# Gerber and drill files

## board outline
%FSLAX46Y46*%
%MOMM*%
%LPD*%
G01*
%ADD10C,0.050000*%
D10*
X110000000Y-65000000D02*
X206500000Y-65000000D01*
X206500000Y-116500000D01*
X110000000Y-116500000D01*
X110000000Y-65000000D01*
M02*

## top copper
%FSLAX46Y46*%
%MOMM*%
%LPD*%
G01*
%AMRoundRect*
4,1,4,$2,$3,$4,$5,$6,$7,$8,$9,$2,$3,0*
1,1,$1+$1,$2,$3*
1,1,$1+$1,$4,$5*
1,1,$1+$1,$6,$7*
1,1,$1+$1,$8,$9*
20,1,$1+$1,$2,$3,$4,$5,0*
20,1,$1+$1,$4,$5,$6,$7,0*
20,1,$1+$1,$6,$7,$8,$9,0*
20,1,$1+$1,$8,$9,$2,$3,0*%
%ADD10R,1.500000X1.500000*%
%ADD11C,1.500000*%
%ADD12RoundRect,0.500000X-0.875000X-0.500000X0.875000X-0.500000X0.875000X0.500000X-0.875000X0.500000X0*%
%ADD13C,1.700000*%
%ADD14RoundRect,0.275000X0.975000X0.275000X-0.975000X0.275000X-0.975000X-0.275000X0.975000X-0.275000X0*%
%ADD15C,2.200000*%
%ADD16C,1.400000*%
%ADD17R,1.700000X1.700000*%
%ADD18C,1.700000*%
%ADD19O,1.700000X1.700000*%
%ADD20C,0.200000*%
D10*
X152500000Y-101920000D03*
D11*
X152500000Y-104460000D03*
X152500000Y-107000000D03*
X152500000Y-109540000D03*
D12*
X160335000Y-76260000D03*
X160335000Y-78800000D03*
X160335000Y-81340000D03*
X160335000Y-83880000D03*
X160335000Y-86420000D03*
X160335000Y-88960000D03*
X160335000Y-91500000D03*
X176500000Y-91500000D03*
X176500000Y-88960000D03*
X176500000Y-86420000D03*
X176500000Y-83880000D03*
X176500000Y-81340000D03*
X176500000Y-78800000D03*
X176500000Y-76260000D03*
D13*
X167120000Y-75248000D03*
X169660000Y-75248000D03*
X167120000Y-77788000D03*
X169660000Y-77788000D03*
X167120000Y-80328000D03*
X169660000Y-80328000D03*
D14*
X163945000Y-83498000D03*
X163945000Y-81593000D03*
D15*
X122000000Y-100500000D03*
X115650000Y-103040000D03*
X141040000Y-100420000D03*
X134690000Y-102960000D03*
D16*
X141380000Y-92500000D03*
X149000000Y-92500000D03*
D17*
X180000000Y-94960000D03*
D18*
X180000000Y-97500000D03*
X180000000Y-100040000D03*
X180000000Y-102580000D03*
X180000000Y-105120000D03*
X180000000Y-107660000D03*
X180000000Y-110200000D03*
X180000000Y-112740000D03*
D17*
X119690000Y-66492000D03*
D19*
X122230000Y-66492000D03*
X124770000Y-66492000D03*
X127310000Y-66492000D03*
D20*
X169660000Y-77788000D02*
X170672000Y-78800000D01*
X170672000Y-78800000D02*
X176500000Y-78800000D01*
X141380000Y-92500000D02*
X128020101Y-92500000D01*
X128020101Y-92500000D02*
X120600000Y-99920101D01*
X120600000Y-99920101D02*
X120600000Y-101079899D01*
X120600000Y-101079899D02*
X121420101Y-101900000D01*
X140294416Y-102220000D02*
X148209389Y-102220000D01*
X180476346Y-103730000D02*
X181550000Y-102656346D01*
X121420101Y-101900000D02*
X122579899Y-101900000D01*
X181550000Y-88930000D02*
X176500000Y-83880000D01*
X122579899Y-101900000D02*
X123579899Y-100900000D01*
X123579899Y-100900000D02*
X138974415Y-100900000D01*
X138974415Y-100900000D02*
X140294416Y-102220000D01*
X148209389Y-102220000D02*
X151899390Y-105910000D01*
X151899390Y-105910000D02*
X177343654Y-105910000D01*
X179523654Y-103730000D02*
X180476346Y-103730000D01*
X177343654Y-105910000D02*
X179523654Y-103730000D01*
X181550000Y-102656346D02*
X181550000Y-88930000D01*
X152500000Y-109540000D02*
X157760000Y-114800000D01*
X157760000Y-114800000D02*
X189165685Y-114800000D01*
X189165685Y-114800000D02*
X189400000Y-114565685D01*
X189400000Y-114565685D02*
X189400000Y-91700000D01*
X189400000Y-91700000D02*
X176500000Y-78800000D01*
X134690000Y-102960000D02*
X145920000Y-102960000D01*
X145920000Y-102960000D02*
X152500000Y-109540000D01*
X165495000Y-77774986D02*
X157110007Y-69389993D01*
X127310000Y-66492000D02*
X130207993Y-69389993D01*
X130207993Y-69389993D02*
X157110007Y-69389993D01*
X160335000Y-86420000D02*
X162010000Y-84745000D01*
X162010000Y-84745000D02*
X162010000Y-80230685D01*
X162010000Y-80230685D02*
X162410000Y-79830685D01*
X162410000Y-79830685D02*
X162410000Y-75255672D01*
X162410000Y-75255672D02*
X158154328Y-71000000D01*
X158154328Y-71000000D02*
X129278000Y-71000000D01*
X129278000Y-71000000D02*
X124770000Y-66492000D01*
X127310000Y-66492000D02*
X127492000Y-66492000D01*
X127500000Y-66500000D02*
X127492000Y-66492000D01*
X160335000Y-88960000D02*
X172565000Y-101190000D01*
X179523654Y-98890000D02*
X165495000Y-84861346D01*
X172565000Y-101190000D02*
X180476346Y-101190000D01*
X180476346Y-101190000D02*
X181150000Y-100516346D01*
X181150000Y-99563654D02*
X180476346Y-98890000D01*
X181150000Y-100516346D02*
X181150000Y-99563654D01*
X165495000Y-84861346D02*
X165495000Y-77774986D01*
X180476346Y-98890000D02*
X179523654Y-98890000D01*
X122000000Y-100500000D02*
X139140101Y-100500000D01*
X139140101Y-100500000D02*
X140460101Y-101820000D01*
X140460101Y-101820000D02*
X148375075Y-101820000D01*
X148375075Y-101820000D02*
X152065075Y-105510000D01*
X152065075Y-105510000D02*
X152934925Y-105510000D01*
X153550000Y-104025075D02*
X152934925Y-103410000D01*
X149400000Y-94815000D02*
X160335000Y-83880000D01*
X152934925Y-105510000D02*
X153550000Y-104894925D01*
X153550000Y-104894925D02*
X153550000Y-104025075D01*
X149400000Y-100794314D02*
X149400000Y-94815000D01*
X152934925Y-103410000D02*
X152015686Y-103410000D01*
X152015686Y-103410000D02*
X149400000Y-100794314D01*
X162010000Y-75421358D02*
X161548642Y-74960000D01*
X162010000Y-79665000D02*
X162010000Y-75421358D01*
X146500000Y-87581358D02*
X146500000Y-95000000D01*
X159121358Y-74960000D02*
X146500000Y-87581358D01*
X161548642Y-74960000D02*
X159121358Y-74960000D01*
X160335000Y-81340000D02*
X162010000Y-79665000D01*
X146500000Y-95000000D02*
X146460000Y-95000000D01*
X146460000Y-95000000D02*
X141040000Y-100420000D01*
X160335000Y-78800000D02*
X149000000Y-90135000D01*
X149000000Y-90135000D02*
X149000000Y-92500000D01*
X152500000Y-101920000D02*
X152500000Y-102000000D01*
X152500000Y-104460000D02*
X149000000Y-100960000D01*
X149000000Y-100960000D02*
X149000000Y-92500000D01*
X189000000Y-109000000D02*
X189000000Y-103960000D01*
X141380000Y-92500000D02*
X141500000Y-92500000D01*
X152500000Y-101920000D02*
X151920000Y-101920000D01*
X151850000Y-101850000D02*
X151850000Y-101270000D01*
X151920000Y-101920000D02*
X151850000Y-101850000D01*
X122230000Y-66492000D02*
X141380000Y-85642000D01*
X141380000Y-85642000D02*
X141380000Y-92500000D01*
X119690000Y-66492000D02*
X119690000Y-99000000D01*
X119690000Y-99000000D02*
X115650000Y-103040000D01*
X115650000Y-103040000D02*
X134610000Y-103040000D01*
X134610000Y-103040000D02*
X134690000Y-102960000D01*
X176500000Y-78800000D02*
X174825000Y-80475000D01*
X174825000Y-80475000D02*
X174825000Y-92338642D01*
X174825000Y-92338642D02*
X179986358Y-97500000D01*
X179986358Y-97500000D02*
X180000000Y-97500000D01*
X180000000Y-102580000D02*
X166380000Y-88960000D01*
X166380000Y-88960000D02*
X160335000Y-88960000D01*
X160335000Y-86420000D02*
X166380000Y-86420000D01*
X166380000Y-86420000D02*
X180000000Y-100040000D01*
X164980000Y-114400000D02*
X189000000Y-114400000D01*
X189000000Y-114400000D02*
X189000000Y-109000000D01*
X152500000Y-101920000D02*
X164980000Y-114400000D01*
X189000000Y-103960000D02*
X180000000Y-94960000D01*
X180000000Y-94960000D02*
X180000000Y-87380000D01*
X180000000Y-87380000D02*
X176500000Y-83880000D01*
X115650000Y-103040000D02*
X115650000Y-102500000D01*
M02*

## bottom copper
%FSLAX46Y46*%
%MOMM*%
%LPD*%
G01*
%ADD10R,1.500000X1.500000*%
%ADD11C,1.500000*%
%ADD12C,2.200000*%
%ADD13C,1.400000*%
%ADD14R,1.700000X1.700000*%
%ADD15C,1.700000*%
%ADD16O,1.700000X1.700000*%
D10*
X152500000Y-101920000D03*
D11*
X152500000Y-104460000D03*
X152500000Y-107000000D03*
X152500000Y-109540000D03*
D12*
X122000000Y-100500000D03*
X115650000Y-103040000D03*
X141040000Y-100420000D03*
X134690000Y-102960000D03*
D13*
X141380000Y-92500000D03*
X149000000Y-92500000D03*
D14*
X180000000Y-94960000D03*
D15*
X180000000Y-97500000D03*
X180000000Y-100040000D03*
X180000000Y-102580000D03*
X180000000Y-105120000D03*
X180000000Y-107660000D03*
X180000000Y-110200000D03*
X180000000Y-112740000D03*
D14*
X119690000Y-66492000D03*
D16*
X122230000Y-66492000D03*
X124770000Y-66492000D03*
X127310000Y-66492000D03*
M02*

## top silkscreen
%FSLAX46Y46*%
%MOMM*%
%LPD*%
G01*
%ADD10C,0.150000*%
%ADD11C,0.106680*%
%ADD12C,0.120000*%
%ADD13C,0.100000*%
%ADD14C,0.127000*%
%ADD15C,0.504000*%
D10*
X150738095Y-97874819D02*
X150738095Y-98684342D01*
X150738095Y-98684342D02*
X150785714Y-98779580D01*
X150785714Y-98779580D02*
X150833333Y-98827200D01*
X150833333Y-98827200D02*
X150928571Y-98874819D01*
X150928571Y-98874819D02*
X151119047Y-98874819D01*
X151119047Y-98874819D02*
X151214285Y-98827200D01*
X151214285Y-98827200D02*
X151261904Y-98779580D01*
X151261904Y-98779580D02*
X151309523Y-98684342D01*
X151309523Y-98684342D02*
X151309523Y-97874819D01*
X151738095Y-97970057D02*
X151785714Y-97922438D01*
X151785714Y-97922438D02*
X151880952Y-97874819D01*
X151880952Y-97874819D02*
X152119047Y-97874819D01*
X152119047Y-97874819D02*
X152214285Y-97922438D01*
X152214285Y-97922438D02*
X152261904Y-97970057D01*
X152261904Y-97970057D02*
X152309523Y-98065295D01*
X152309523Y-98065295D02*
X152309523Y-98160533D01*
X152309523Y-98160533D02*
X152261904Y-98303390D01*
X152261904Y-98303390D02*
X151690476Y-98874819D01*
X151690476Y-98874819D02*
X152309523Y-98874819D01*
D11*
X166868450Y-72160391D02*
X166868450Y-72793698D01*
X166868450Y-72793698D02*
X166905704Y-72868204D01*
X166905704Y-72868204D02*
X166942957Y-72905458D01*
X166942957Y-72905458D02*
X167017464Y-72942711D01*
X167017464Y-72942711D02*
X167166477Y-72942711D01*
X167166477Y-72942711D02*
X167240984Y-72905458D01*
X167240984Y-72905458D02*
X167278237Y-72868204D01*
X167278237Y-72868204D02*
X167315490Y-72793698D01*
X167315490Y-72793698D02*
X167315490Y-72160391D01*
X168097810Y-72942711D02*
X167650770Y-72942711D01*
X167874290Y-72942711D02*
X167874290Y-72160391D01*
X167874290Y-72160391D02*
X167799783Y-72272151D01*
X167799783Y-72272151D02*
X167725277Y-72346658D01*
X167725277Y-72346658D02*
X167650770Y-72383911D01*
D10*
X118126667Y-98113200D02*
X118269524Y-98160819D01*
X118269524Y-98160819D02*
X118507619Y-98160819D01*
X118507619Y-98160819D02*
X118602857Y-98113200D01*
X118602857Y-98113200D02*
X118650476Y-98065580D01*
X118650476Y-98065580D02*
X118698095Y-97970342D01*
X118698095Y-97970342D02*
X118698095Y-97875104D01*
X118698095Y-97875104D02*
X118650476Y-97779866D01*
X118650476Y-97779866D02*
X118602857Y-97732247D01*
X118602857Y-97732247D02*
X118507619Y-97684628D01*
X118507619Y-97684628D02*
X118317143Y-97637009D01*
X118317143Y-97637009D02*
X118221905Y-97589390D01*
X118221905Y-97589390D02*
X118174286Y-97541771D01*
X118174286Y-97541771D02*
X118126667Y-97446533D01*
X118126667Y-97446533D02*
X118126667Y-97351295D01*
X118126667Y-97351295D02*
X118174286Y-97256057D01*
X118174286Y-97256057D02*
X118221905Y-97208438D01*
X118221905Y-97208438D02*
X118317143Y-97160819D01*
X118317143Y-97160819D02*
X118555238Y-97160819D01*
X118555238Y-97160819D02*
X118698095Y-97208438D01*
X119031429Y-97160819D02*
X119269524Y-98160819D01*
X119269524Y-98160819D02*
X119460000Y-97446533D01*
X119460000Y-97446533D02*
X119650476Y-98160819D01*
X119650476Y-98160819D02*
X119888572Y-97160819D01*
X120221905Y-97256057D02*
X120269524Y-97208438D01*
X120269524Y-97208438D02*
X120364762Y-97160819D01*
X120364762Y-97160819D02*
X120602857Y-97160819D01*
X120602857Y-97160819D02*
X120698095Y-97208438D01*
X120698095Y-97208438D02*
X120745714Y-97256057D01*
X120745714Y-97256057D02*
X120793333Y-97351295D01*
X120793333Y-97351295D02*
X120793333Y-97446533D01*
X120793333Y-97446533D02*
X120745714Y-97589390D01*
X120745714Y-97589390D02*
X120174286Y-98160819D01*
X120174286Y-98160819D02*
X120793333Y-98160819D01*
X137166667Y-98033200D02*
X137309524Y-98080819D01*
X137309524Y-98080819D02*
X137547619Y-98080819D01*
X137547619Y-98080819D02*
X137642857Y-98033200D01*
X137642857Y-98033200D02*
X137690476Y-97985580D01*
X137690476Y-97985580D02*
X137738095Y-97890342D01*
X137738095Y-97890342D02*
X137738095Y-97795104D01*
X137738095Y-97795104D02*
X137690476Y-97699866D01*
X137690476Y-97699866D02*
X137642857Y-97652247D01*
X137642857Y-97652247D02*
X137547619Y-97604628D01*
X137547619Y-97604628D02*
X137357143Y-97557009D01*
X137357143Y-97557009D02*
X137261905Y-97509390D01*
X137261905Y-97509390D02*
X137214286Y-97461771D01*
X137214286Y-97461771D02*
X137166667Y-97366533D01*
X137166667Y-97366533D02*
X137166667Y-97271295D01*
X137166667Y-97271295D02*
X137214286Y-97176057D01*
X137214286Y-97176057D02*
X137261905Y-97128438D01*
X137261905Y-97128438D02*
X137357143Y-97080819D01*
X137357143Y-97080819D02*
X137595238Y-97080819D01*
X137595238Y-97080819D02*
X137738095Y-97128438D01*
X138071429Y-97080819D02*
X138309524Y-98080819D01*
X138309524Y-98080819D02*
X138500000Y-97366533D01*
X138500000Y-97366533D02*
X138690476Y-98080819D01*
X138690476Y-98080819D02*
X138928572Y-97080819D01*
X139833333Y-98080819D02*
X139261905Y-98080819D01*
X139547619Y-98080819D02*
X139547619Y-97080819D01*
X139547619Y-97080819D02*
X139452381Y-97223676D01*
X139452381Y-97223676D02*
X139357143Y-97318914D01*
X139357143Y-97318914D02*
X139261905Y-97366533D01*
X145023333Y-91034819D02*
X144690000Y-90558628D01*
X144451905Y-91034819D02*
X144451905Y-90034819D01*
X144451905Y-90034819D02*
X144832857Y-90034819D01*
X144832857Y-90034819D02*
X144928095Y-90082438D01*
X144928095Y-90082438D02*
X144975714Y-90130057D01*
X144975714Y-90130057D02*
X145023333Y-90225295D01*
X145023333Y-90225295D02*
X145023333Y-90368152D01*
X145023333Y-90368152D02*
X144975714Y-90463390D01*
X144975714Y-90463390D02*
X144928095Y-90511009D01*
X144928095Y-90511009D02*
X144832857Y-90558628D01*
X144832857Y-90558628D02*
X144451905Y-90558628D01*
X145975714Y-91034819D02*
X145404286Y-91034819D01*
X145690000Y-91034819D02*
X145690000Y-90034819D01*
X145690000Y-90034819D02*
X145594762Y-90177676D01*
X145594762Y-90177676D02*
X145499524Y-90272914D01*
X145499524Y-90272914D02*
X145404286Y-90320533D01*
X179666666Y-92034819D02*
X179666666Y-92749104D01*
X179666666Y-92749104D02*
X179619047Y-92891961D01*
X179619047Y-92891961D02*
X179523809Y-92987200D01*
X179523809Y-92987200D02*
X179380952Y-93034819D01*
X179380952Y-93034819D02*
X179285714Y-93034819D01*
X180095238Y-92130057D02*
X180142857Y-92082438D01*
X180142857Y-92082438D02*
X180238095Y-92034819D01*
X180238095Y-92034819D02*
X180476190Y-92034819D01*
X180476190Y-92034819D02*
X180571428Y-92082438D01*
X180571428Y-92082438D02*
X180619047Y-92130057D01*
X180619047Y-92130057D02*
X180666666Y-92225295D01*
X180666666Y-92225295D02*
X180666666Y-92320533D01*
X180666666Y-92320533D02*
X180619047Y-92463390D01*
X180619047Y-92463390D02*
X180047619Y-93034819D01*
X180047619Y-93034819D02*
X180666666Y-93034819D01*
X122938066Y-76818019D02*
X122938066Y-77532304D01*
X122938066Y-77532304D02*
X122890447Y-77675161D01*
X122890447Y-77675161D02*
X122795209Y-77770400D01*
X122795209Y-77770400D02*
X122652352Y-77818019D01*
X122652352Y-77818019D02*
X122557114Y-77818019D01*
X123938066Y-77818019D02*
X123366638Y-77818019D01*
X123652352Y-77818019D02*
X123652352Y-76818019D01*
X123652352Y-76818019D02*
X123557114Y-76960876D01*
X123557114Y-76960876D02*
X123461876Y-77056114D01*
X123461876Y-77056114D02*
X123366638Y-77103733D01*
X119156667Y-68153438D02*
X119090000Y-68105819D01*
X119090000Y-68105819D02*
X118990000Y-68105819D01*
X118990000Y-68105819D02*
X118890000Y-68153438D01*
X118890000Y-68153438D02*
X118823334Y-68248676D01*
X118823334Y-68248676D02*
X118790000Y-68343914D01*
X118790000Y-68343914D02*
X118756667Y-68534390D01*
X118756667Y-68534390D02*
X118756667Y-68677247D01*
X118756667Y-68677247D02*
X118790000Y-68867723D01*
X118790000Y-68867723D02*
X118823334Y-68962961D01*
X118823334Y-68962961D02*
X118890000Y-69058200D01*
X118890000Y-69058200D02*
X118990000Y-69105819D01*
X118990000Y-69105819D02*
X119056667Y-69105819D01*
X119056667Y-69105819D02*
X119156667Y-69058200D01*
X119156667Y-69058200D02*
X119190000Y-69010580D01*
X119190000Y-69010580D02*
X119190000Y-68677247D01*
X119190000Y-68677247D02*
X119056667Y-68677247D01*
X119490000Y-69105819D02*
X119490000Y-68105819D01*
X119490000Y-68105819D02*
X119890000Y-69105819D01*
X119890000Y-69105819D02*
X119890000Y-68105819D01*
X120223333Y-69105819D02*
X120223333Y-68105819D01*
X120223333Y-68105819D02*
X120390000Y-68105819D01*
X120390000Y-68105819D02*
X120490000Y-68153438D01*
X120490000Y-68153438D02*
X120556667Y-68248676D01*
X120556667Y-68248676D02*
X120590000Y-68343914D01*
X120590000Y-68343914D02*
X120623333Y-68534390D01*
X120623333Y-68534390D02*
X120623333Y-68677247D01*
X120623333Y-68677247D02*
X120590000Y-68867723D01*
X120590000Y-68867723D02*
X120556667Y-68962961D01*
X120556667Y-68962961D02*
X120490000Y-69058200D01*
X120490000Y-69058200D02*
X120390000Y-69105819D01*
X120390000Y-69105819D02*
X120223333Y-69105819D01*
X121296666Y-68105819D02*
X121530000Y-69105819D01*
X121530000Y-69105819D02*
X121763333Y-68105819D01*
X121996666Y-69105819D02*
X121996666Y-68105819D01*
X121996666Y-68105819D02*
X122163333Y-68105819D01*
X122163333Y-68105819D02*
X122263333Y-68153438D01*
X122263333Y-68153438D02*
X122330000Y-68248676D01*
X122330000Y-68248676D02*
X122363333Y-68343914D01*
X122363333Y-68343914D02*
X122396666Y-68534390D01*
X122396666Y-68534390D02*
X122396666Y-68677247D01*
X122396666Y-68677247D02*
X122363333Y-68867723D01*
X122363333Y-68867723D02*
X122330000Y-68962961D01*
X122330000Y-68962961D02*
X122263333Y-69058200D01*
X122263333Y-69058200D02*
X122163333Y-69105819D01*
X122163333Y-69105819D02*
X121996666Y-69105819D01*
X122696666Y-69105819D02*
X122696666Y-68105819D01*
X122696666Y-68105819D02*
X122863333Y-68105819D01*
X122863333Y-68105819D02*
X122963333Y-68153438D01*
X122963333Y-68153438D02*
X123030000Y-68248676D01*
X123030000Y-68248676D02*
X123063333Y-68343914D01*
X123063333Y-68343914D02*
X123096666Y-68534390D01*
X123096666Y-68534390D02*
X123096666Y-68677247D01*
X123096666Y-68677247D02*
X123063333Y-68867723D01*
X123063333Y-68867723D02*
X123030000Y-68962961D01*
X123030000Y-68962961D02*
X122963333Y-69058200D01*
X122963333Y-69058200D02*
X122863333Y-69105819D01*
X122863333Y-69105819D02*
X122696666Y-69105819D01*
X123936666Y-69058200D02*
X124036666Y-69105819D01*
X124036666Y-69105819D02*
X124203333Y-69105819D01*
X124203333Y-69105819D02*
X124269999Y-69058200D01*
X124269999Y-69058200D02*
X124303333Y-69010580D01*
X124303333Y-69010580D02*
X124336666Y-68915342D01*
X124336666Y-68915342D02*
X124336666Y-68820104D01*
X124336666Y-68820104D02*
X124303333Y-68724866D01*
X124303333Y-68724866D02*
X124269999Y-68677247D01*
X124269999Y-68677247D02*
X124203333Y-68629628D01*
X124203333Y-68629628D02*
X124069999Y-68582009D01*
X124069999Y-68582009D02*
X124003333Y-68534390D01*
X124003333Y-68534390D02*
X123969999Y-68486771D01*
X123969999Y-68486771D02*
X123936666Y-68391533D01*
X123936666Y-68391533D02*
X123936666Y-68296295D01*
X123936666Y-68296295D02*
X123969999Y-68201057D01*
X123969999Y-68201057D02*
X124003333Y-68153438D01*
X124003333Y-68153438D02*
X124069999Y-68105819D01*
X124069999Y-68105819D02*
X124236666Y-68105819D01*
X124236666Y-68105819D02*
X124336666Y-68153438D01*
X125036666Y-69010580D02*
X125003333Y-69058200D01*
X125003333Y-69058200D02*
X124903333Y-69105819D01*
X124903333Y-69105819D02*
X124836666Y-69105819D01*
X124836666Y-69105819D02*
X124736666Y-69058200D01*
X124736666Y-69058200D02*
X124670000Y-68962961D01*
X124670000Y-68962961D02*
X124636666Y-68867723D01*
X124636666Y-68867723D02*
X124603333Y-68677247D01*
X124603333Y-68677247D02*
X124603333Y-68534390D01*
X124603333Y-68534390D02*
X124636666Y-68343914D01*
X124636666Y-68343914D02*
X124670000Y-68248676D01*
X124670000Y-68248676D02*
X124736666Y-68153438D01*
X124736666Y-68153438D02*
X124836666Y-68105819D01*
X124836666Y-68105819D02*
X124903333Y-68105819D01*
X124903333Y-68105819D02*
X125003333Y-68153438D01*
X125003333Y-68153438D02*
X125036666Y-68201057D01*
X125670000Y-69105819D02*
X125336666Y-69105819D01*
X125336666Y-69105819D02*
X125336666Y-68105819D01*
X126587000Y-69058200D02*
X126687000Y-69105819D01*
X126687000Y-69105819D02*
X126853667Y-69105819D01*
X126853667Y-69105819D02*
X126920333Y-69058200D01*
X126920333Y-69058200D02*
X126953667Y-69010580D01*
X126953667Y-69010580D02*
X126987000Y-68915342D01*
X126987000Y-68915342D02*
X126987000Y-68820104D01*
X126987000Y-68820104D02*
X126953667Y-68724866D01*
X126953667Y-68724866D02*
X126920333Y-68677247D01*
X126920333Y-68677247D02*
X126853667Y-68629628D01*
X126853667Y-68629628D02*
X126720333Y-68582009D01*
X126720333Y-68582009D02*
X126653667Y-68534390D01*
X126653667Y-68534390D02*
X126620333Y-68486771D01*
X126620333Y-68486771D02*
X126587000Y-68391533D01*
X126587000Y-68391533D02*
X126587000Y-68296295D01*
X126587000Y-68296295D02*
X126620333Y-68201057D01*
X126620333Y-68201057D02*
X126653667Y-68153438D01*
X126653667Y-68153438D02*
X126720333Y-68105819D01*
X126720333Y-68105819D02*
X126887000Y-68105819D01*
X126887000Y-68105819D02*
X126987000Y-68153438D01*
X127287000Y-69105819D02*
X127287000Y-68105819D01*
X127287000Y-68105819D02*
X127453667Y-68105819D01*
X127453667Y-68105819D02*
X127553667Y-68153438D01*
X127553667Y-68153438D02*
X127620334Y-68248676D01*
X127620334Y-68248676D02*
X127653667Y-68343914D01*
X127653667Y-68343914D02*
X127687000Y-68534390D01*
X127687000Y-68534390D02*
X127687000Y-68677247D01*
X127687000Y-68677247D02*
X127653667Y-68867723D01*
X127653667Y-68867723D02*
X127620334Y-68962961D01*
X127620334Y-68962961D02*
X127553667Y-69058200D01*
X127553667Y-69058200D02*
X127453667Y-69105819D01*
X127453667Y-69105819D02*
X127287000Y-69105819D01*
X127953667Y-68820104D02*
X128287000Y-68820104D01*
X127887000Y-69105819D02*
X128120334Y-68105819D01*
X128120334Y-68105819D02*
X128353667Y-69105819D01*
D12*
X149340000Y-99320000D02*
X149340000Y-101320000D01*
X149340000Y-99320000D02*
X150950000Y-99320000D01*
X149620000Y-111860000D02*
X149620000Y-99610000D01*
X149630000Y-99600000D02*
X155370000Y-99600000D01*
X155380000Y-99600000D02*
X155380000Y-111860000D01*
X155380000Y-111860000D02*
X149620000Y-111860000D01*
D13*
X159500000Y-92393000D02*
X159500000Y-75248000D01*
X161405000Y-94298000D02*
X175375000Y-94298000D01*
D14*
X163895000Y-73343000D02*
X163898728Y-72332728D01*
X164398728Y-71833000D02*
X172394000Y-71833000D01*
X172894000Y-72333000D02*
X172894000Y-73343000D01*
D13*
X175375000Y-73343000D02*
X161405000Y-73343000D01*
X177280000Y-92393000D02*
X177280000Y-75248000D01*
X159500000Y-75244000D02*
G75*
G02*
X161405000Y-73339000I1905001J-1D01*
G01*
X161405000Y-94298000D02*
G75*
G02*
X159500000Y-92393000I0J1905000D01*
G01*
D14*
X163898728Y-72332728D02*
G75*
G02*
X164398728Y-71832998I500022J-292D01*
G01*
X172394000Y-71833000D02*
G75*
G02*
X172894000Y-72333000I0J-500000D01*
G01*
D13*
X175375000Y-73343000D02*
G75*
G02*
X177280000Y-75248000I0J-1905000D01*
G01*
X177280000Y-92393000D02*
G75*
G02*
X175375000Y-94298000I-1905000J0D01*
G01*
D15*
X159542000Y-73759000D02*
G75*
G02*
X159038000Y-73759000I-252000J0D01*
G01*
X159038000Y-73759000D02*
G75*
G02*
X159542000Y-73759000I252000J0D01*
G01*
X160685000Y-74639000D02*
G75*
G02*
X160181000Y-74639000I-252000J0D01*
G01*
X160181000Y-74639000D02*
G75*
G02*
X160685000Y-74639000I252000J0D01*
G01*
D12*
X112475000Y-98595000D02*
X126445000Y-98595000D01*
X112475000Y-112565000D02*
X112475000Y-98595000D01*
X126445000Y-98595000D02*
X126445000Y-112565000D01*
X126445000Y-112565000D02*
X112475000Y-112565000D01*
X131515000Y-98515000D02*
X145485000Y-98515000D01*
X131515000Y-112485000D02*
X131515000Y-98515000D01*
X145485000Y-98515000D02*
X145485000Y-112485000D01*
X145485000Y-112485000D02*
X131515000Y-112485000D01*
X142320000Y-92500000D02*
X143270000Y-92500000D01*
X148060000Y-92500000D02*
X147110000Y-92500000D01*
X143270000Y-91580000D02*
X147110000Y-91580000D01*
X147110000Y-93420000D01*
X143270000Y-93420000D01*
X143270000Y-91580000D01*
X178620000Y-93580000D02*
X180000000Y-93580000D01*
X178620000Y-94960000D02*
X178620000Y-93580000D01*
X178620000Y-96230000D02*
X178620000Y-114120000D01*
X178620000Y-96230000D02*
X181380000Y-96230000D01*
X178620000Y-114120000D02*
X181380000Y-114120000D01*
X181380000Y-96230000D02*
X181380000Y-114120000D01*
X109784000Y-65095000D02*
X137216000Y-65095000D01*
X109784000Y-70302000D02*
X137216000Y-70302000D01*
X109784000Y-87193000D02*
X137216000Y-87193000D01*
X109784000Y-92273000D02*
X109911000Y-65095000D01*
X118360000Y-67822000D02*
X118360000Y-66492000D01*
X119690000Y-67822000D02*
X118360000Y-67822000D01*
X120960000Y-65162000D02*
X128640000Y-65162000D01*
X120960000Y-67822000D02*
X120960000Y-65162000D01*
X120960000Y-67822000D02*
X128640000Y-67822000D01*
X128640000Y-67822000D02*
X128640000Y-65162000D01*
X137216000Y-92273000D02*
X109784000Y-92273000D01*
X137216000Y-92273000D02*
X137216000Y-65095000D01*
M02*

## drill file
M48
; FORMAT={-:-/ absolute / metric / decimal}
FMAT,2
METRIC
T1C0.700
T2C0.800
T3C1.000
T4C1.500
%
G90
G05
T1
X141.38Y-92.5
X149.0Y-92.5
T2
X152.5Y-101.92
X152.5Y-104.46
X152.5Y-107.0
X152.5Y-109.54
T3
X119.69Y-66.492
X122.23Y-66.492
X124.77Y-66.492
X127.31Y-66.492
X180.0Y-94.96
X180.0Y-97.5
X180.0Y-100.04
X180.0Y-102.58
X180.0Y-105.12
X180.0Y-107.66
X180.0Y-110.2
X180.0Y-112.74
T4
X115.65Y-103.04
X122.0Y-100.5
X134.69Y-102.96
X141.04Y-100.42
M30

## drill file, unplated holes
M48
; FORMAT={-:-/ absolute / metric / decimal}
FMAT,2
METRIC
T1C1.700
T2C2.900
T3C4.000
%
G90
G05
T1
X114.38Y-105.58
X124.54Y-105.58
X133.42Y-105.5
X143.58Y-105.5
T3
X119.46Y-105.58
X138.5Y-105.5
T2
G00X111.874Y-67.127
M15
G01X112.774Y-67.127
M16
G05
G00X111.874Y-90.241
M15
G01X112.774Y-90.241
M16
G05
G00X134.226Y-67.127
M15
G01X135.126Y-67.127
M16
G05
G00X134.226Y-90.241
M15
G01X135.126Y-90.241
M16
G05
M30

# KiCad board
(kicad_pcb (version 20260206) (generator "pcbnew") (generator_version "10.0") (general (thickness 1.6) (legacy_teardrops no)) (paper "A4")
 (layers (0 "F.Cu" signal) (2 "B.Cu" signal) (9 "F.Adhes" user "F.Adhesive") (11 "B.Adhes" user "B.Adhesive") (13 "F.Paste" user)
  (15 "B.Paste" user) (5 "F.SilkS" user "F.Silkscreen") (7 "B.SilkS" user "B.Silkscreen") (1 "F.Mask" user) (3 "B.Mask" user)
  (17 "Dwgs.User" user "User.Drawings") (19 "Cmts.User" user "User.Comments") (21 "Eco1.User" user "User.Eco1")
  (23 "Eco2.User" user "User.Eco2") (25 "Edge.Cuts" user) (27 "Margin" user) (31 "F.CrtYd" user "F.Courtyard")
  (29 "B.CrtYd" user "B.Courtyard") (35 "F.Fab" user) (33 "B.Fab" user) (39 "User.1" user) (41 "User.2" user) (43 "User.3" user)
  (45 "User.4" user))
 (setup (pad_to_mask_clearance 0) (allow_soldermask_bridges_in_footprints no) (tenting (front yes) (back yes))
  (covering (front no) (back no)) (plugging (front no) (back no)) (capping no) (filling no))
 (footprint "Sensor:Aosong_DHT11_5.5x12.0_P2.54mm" (layer "F.Cu") (at 152.5 101.92)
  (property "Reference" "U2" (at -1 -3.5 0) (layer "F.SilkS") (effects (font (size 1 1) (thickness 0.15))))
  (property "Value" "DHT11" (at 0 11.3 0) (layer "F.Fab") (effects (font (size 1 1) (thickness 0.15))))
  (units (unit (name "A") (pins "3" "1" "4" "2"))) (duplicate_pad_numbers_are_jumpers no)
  (fp_line (start -3.16 -2.6) (end -3.16 -0.6) (stroke (width 0.12) (type solid)) (layer "F.SilkS"))
  (fp_line (start -3.16 -2.6) (end -1.55 -2.6) (stroke (width 0.12) (type solid)) (layer "F.SilkS"))
  (fp_line (start -2.88 9.94) (end -2.88 -2.31) (stroke (width 0.12) (type solid)) (layer "F.SilkS"))
  (fp_line (start -2.87 -2.32) (end 2.87 -2.32) (stroke (width 0.12) (type solid)) (layer "F.SilkS"))
  (fp_line (start 2.88 -2.32) (end 2.88 9.94) (stroke (width 0.12) (type solid)) (layer "F.SilkS"))
  (fp_line (start 2.88 9.94) (end -2.88 9.94) (stroke (width 0.12) (type solid)) (layer "F.SilkS"))
  (pad "1" thru_hole rect (at 0 0) (size 1.5 1.5) (drill 0.8) (layers "*.Cu" "*.Mask") (remove_unused_layers no) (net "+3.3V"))
  (pad "2" thru_hole circle (at 0 2.54) (size 1.5 1.5) (drill 0.8) (layers "*.Cu" "*.Mask") (remove_unused_layers no) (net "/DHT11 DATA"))
  (pad "3" thru_hole circle (at 0 5.08) (size 1.5 1.5) (drill 0.8) (layers "*.Cu" "*.Mask") (remove_unused_layers no)
   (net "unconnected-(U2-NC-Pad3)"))
  (pad "4" thru_hole circle (at 0 7.62) (size 1.5 1.5) (drill 0.8) (layers "*.Cu" "*.Mask") (remove_unused_layers no) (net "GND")))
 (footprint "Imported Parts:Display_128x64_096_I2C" (layer "F.Cu") (at 123.5 66.492)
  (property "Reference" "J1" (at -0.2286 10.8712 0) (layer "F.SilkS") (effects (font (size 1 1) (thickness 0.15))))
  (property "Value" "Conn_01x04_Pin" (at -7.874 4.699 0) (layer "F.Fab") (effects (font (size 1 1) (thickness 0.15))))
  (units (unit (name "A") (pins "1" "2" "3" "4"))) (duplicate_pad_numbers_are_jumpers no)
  (fp_line (start -13.716 -1.397) (end 13.716 -1.397) (stroke (width 0.12) (type solid)) (layer "F.SilkS"))
  (fp_line (start -13.716 3.81) (end 13.716 3.81) (stroke (width 0.12) (type solid)) (layer "F.SilkS"))
  (fp_line (start -13.716 20.701) (end 13.716 20.701) (stroke (width 0.12) (type solid)) (layer "F.SilkS"))
  (fp_line (start -13.716 25.781) (end -13.589 -1.397) (stroke (width 0.12) (type solid)) (layer "F.SilkS"))
  (fp_line (start -5.14 1.33) (end -5.14 0) (stroke (width 0.12) (type solid)) (layer "F.SilkS"))
  (fp_line (start -3.81 1.33) (end -5.14 1.33) (stroke (width 0.12) (type solid)) (layer "F.SilkS"))
  (fp_line (start -2.54 -1.33) (end 5.14 -1.33) (stroke (width 0.12) (type solid)) (layer "F.SilkS"))
  (fp_line (start -2.54 1.33) (end -2.54 -1.33) (stroke (width 0.12) (type solid)) (layer "F.SilkS"))
  (fp_line (start -2.54 1.33) (end 5.14 1.33) (stroke (width 0.12) (type solid)) (layer "F.SilkS"))
  (fp_line (start 5.14 1.33) (end 5.14 -1.33) (stroke (width 0.12) (type solid)) (layer "F.SilkS"))
  (fp_line (start 13.716 25.781) (end -13.716 25.781) (stroke (width 0.12) (type solid)) (layer "F.SilkS"))
  (fp_line (start 13.716 25.781) (end 13.716 -1.397) (stroke (width 0.12) (type solid)) (layer "F.SilkS"))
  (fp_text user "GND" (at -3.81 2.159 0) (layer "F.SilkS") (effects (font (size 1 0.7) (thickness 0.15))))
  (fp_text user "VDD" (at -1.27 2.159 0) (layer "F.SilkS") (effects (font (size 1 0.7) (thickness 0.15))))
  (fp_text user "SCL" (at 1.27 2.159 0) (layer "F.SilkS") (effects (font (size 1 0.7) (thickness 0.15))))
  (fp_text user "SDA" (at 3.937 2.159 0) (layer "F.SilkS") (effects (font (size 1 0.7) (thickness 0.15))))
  (pad "" np_thru_hole oval (at -11.176 0.635) (size 3.8 2.9) (drill oval 3.8 2.9) (layers "*.Cu" "*.Mask"))
  (pad "" np_thru_hole oval (at -11.176 23.749) (size 3.8 2.9) (drill oval 3.8 2.9) (layers "*.Cu" "*.Mask"))
  (pad "" np_thru_hole oval (at 11.176 0.635) (size 3.8 2.9) (drill oval 3.8 2.9) (layers "*.Cu" "*.Mask"))
  (pad "" np_thru_hole oval (at 11.176 23.749) (size 3.8 2.9) (drill oval 3.8 2.9) (layers "*.Cu" "*.Mask"))
  (pad "1" thru_hole rect (at -3.81 0 90) (size 1.7 1.7) (drill 1) (layers "*.Cu" "*.Mask") (remove_unused_layers no) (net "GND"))
  (pad "2" thru_hole oval (at -1.27 0 90) (size 1.7 1.7) (drill 1) (layers "*.Cu" "*.Mask") (remove_unused_layers no) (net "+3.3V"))
  (pad "3" thru_hole oval (at 1.27 0 90) (size 1.7 1.7) (drill 1) (layers "*.Cu" "*.Mask") (remove_unused_layers no) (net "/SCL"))
  (pad "4" thru_hole oval (at 3.81 0 90) (size 1.7 1.7) (drill 1) (layers "*.Cu" "*.Mask") (remove_unused_layers no) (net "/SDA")))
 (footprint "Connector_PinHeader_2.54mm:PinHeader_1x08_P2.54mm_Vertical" (layer "F.Cu") (at 180 94.96)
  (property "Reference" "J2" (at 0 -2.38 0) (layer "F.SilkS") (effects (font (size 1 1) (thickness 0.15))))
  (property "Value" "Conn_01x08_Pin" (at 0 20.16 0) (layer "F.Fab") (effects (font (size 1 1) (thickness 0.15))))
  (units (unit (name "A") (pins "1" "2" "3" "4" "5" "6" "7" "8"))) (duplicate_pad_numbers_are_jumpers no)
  (fp_line (start -1.38 -1.38) (end 0 -1.38) (stroke (width 0.12) (type solid)) (layer "F.SilkS"))
  (fp_line (start -1.38 0) (end -1.38 -1.38) (stroke (width 0.12) (type solid)) (layer "F.SilkS"))
  (fp_line (start -1.38 1.27) (end -1.38 19.16) (stroke (width 0.12) (type solid)) (layer "F.SilkS"))
  (fp_line (start -1.38 1.27) (end 1.38 1.27) (stroke (width 0.12) (type solid)) (layer "F.SilkS"))
  (fp_line (start -1.38 19.16) (end 1.38 19.16) (stroke (width 0.12) (type solid)) (layer "F.SilkS"))
  (fp_line (start 1.38 1.27) (end 1.38 19.16) (stroke (width 0.12) (type solid)) (layer "F.SilkS"))
  (pad "1" thru_hole rect (at 0 0) (size 1.7 1.7) (drill 1) (layers "*.Cu" "*.Mask") (remove_unused_layers no) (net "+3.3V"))
  (pad "2" thru_hole circle (at 0 2.54) (size 1.7 1.7) (drill 1) (layers "*.Cu" "*.Mask") (remove_unused_layers no) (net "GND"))
  (pad "3" thru_hole circle (at 0 5.08) (size 1.7 1.7) (drill 1) (layers "*.Cu" "*.Mask") (remove_unused_layers no) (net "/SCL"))
  (pad "4" thru_hole circle (at 0 7.62) (size 1.7 1.7) (drill 1) (layers "*.Cu" "*.Mask") (remove_unused_layers no) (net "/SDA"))
  (pad "5" thru_hole circle (at 0 10.16) (size 1.7 1.7) (drill 1) (layers "*.Cu" "*.Mask") (remove_unused_layers no)
   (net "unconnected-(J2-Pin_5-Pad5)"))
  (pad "6" thru_hole circle (at 0 12.7) (size 1.7 1.7) (drill 1) (layers "*.Cu" "*.Mask") (remove_unused_layers no)
   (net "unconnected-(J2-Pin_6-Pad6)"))
  (pad "7" thru_hole circle (at 0 15.24) (size 1.7 1.7) (drill 1) (layers "*.Cu" "*.Mask") (remove_unused_layers no)
   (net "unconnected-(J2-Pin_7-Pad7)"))
  (pad "8" thru_hole circle (at 0 17.78) (size 1.7 1.7) (drill 1) (layers "*.Cu" "*.Mask") (remove_unused_layers no)
   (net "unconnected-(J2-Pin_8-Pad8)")))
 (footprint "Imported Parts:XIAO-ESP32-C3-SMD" (layer "F.Cu") (at 159.5 94.38)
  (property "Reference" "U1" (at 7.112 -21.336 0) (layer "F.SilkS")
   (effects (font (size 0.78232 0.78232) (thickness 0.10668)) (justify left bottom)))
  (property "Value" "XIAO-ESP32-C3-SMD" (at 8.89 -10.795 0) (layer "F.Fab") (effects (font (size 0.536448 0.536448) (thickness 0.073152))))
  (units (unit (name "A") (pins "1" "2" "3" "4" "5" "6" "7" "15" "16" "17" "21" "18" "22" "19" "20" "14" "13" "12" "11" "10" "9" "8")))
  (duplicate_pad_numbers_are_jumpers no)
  (fp_line (start 0 -1.987) (end 0 -19.132) (stroke (width 0.1) (type solid)) (layer "F.SilkS"))
  (fp_line (start 1.905 -0.082) (end 15.875 -0.082) (stroke (width 0.1) (type solid)) (layer "F.SilkS"))
  (fp_line (start 4.395 -21.037) (end 4.398728 -22.047272) (stroke (width 0.127) (type solid)) (layer "F.SilkS"))
  (fp_line (start 4.898728 -22.547) (end 12.894 -22.547) (stroke (width 0.127) (type solid)) (layer "F.SilkS"))
  (fp_line (start 13.394 -22.047) (end 13.394 -21.037) (stroke (width 0.127) (type solid)) (layer "F.SilkS"))
  (fp_line (start 15.875 -21.037) (end 1.905 -21.037) (stroke (width 0.1) (type solid)) (layer "F.SilkS"))
  (fp_line (start 17.78 -1.987) (end 17.78 -19.132) (stroke (width 0.1) (type solid)) (layer "F.SilkS"))
  (fp_arc (start 0 -19.136) (mid 0.557962 -20.483038) (end 1.905 -21.041) (stroke (width 0.1) (type solid)) (layer "F.SilkS"))
  (fp_arc (start 1.905 -0.082) (mid 0.557962 -0.639962) (end 0 -1.987) (stroke (width 0.1) (type solid)) (layer "F.SilkS"))
  (fp_arc (start 4.398728 -22.047272) (mid 4.545272 -22.40064) (end 4.898728 -22.547) (stroke (width 0.127) (type default))
   (layer "F.SilkS"))
  (fp_arc (start 12.894 -22.547) (mid 13.247553 -22.400553) (end 13.394 -22.047) (stroke (width 0.127) (type default)) (layer "F.SilkS"))
  (fp_arc (start 15.875 -21.037) (mid 17.222038 -20.479038) (end 17.78 -19.132) (stroke (width 0.1) (type solid)) (layer "F.SilkS"))
  (fp_arc (start 17.78 -1.987) (mid 17.222038 -0.639962) (end 15.875 -0.082) (stroke (width 0.1) (type solid)) (layer "F.SilkS"))
  (fp_circle (center -0.21 -20.621) (end -0.21 -20.875) (stroke (width 0.5) (type solid)) (fill yes) (layer "F.SilkS"))
  (fp_circle (center 0.933 -19.741) (end 0.933 -19.995) (stroke (width 0.5) (type solid)) (fill yes) (layer "F.SilkS"))
  (pad "1" smd roundrect (at 0.835 -18.12) (size 2.75 2) (layers "F.Cu" "F.Mask" "F.Paste") (roundrect_rratio 0.25)
   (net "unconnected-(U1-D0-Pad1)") (solder_mask_margin 0.0508) (thermal_bridge_angle 45))
  (pad "2" smd roundrect (at 0.835 -15.58) (size 2.75 2) (layers "F.Cu" "F.Mask" "F.Paste") (roundrect_rratio 0.25) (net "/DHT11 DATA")
   (solder_mask_margin 0.0508) (thermal_bridge_angle 45))
  (pad "3" smd roundrect (at 0.835 -13.04) (size 2.75 2) (layers "F.Cu" "F.Mask" "F.Paste") (roundrect_rratio 0.25) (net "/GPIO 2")
   (solder_mask_margin 0.0508) (thermal_bridge_angle 45))
  (pad "4" smd roundrect (at 0.835 -10.5) (size 2.75 2) (layers "F.Cu" "F.Mask" "F.Paste") (roundrect_rratio 0.25) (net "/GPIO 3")
   (solder_mask_margin 0.0508) (thermal_bridge_angle 45))
  (pad "5" smd roundrect (at 0.835 -7.96) (size 2.75 2) (layers "F.Cu" "F.Mask" "F.Paste") (roundrect_rratio 0.25) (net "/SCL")
   (solder_mask_margin 0.0508) (thermal_bridge_angle 45))
  (pad "6" smd roundrect (at 0.835 -5.42) (size 2.75 2) (layers "F.Cu" "F.Mask" "F.Paste") (roundrect_rratio 0.25) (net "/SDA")
   (solder_mask_margin 0.0508) (thermal_bridge_angle 45))
  (pad "7" smd roundrect (at 0.835 -2.88) (size 2.75 2) (layers "F.Cu" "F.Mask" "F.Paste") (roundrect_rratio 0.25)
   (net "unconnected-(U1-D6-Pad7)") (solder_mask_margin 0.0508) (thermal_bridge_angle 45))
  (pad "8" smd roundrect (at 17 -2.88) (size 2.75 2) (layers "F.Cu" "F.Mask" "F.Paste") (roundrect_rratio 0.25)
   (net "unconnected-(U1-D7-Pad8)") (solder_mask_margin 0.0508) (thermal_bridge_angle 45))
  (pad "9" smd roundrect (at 17 -5.42) (size 2.75 2) (layers "F.Cu" "F.Mask" "F.Paste") (roundrect_rratio 0.25)
   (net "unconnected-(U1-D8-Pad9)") (solder_mask_margin 0.0508) (thermal_bridge_angle 45))
  (pad "10" smd roundrect (at 17 -7.96) (size 2.75 2) (layers "F.Cu" "F.Mask" "F.Paste") (roundrect_rratio 0.25)
   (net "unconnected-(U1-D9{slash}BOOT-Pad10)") (solder_mask_margin 0.0508) (thermal_bridge_angle 45))
  (pad "11" smd roundrect (at 17 -10.5) (size 2.75 2) (layers "F.Cu" "F.Mask" "F.Paste") (roundrect_rratio 0.25) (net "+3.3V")
   (solder_mask_margin 0.0508) (thermal_bridge_angle 45))
  (pad "12" smd roundrect (at 17 -13.04) (size 2.75 2) (layers "F.Cu" "F.Mask" "F.Paste") (roundrect_rratio 0.25)
   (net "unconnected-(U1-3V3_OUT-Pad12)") (solder_mask_margin 0.0508) (thermal_bridge_angle 45))
  (pad "13" smd roundrect (at 17 -15.58) (size 2.75 2) (layers "F.Cu" "F.Mask" "F.Paste") (roundrect_rratio 0.25) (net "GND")
   (solder_mask_margin 0.0508) (thermal_bridge_angle 45))
  (pad "14" smd roundrect (at 17 -18.12) (size 2.75 2) (layers "F.Cu" "F.Mask" "F.Paste") (roundrect_rratio 0.25) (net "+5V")
   (solder_mask_margin 0.0508) (thermal_bridge_angle 45))
  (pad "15" smd circle (at 7.62 -19.132) (size 1.7 1.7) (layers "F.Cu" "F.Mask" "F.Paste") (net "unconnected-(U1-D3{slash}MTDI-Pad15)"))
  (pad "16" smd circle (at 10.16 -19.132) (size 1.7 1.7) (layers "F.Cu" "F.Mask" "F.Paste") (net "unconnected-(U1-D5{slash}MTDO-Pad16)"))
  (pad "17" smd circle (at 7.62 -16.592) (size 1.7 1.7) (layers "F.Cu" "F.Mask" "F.Paste") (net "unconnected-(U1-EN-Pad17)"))
  (pad "18" smd circle (at 10.16 -16.592) (size 1.7 1.7) (layers "F.Cu" "F.Mask" "F.Paste") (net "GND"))
  (pad "19" smd circle (at 7.62 -14.052) (size 1.7 1.7) (layers "F.Cu" "F.Mask" "F.Paste") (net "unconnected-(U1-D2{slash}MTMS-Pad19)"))
  (pad "20" smd circle (at 10.16 -14.052) (size 1.7 1.7) (layers "F.Cu" "F.Mask" "F.Paste") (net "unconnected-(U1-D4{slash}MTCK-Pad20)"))
  (pad "21" smd roundrect (at 4.445 -10.882 180) (size 2.5 1.1) (layers "F.Cu" "F.Mask" "F.Paste") (roundrect_rratio 0.25)
   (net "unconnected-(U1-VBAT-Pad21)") (thermal_bridge_angle 45))
  (pad "22" smd roundrect (at 4.445 -12.787 180) (size 2.5 1.1) (layers "F.Cu" "F.Mask" "F.Paste") (roundrect_rratio 0.25)
   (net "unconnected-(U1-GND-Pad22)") (thermal_bridge_angle 45)))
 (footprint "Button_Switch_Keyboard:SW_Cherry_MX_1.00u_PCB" (layer "F.Cu") (at 141.04 100.42)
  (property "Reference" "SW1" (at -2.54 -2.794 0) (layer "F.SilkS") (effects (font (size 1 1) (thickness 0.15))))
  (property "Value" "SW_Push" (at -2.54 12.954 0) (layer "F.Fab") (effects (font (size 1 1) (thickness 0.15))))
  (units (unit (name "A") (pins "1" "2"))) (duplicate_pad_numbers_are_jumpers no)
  (fp_line (start -9.525 -1.905) (end 4.445 -1.905) (stroke (width 0.12) (type solid)) (layer "F.SilkS"))
  (fp_line (start -9.525 12.065) (end -9.525 -1.905) (stroke (width 0.12) (type solid)) (layer "F.SilkS"))
  (fp_line (start 4.445 -1.905) (end 4.445 12.065) (stroke (width 0.12) (type solid)) (layer "F.SilkS"))
  (fp_line (start 4.445 12.065) (end -9.525 12.065) (stroke (width 0.12) (type solid)) (layer "F.SilkS"))
  (pad "" np_thru_hole circle (at -7.62 5.08) (size 1.7 1.7) (drill 1.7) (layers "*.Cu" "*.Mask"))
  (pad "" np_thru_hole circle (at -2.54 5.08) (size 4 4) (drill 4) (layers "*.Cu" "*.Mask"))
  (pad "" np_thru_hole circle (at 2.54 5.08) (size 1.7 1.7) (drill 1.7) (layers "*.Cu" "*.Mask"))
  (pad "1" thru_hole circle (at 0 0) (size 2.2 2.2) (drill 1.5) (layers "*.Cu" "*.Mask") (remove_unused_layers no) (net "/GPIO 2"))
  (pad "2" thru_hole circle (at -6.35 2.54) (size 2.2 2.2) (drill 1.5) (layers "*.Cu" "*.Mask") (remove_unused_layers no) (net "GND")))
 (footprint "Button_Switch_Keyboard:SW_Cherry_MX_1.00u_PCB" (layer "F.Cu") (at 122 100.5)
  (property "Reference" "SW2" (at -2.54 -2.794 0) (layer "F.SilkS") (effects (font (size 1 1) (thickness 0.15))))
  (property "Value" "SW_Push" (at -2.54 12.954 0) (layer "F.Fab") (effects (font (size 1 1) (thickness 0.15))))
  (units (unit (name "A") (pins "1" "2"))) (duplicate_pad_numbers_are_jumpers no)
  (fp_line (start -9.525 -1.905) (end 4.445 -1.905) (stroke (width 0.12) (type solid)) (layer "F.SilkS"))
  (fp_line (start -9.525 12.065) (end -9.525 -1.905) (stroke (width 0.12) (type solid)) (layer "F.SilkS"))
  (fp_line (start 4.445 -1.905) (end 4.445 12.065) (stroke (width 0.12) (type solid)) (layer "F.SilkS"))
  (fp_line (start 4.445 12.065) (end -9.525 12.065) (stroke (width 0.12) (type solid)) (layer "F.SilkS"))
  (pad "" np_thru_hole circle (at -7.62 5.08) (size 1.7 1.7) (drill 1.7) (layers "*.Cu" "*.Mask"))
  (pad "" np_thru_hole circle (at -2.54 5.08) (size 4 4) (drill 4) (layers "*.Cu" "*.Mask"))
  (pad "" np_thru_hole circle (at 2.54 5.08) (size 1.7 1.7) (drill 1.7) (layers "*.Cu" "*.Mask"))
  (pad "1" thru_hole circle (at 0 0) (size 2.2 2.2) (drill 1.5) (layers "*.Cu" "*.Mask") (remove_unused_layers no) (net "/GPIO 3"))
  (pad "2" thru_hole circle (at -6.35 2.54) (size 2.2 2.2) (drill 1.5) (layers "*.Cu" "*.Mask") (remove_unused_layers no) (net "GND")))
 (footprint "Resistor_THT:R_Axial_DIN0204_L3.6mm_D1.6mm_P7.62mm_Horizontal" (layer "F.Cu") (at 141.38 92.5)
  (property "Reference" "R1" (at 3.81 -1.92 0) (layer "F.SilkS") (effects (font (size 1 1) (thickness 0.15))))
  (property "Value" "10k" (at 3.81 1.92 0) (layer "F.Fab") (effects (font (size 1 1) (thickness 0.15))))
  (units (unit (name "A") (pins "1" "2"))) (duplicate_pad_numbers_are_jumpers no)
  (fp_line (start 0.94 0) (end 1.89 0) (stroke (width 0.12) (type solid)) (layer "F.SilkS"))
  (fp_line (start 6.68 0) (end 5.73 0) (stroke (width 0.12) (type solid)) (layer "F.SilkS"))
  (fp_rect (start 1.89 -0.92) (end 5.73 0.92) (stroke (width 0.12) (type solid)) (fill no) (layer "F.SilkS"))
  (pad "1" thru_hole circle (at 0 0) (size 1.4 1.4) (drill 0.7) (layers "*.Cu" "*.Mask") (remove_unused_layers no) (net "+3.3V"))
  (pad "2" thru_hole circle (at 7.62 0) (size 1.4 1.4) (drill 0.7) (layers "*.Cu" "*.Mask") (remove_unused_layers no) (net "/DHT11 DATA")))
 (gr_rect (start 110 65) (end 206.5 116.5) (stroke (width 0.05) (type default)) (fill no) (layer "Edge.Cuts"))
 (segment (start 141.38 92.5) (end 141.5 92.5) (width 0.2) (layer "F.Cu") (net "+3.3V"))
 (segment (start 179.523654 103.73) (end 180.476346 103.73) (width 0.2) (layer "F.Cu") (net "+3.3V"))
 (segment (start 120.6 101.079899) (end 121.420101 101.9) (width 0.2) (layer "F.Cu") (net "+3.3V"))
 (segment (start 121.420101 101.9) (end 122.579899 101.9) (width 0.2) (layer "F.Cu") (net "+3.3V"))
 (segment (start 151.92 101.92) (end 151.85 101.85) (width 0.2) (layer "F.Cu") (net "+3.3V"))
 (segment (start 141.38 92.5) (end 128.020101 92.5) (width 0.2) (layer "F.Cu") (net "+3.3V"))
 (segment (start 189 114.4) (end 189 109) (width 0.2) (layer "F.Cu") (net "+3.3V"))
 (segment (start 181.55 88.93) (end 176.5 83.88) (width 0.2) (layer "F.Cu") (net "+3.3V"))
 (segment (start 152.5 101.92) (end 152.5 102) (width 0.2) (layer "F.Cu") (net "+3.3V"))
 (segment (start 151.85 101.85) (end 151.85 101.27) (width 0.2) (layer "F.Cu") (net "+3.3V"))
 (segment (start 180 87.38) (end 176.5 83.88) (width 0.2) (layer "F.Cu") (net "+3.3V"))
 (segment (start 189 103.96) (end 180 94.96) (width 0.2) (layer "F.Cu") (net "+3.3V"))
 (segment (start 180 94.96) (end 180 87.38) (width 0.2) (layer "F.Cu") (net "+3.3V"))
 (segment (start 120.6 99.920101) (end 120.6 101.079899) (width 0.2) (layer "F.Cu") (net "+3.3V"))
 (segment (start 181.55 102.656346) (end 181.55 88.93) (width 0.2) (layer "F.Cu") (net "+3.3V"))
 (segment (start 141.38 85.642) (end 141.38 92.5) (width 0.2) (layer "F.Cu") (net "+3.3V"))
 (segment (start 151.89939 105.91) (end 177.343654 105.91) (width 0.2) (layer "F.Cu") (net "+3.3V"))
 (segment (start 152.5 101.92) (end 164.98 114.4) (width 0.2) (layer "F.Cu") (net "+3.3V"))
 (segment (start 140.294416 102.22) (end 148.209389 102.22) (width 0.2) (layer "F.Cu") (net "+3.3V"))
 (segment (start 152.5 101.92) (end 151.92 101.92) (width 0.2) (layer "F.Cu") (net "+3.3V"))
 (segment (start 128.020101 92.5) (end 120.6 99.920101) (width 0.2) (layer "F.Cu") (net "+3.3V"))
 (segment (start 122.579899 101.9) (end 123.579899 100.9) (width 0.2) (layer "F.Cu") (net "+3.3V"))
 (segment (start 180.476346 103.73) (end 181.55 102.656346) (width 0.2) (layer "F.Cu") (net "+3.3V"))
 (segment (start 138.974415 100.9) (end 140.294416 102.22) (width 0.2) (layer "F.Cu") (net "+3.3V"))
 (segment (start 164.98 114.4) (end 189 114.4) (width 0.2) (layer "F.Cu") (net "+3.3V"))
 (segment (start 177.343654 105.91) (end 179.523654 103.73) (width 0.2) (layer "F.Cu") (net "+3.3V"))
 (segment (start 189 109) (end 189 103.96) (width 0.2) (layer "F.Cu") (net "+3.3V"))
 (segment (start 122.23 66.492) (end 141.38 85.642) (width 0.2) (layer "F.Cu") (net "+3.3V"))
 (segment (start 148.209389 102.22) (end 151.89939 105.91) (width 0.2) (layer "F.Cu") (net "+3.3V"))
 (segment (start 123.579899 100.9) (end 138.974415 100.9) (width 0.2) (layer "F.Cu") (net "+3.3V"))
 (segment (start 189.4 91.7) (end 176.5 78.8) (width 0.2) (layer "F.Cu") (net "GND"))
 (segment (start 179.986358 97.5) (end 180 97.5) (width 0.2) (layer "F.Cu") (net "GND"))
 (segment (start 145.92 102.96) (end 152.5 109.54) (width 0.2) (layer "F.Cu") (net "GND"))
 (segment (start 174.825 92.338642) (end 179.986358 97.5) (width 0.2) (layer "F.Cu") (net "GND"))
 (segment (start 157.76 114.8) (end 189.165685 114.8) (width 0.2) (layer "F.Cu") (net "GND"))
 (segment (start 134.69 102.96) (end 145.92 102.96) (width 0.2) (layer "F.Cu") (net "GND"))
 (segment (start 119.69 99) (end 115.65 103.04) (width 0.2) (layer "F.Cu") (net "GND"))
 (segment (start 115.65 103.04) (end 134.61 103.04) (width 0.2) (layer "F.Cu") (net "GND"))
 (segment (start 176.5 78.8) (end 174.825 80.475) (width 0.2) (layer "F.Cu") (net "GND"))
 (segment (start 134.61 103.04) (end 134.69 102.96) (width 0.2) (layer "F.Cu") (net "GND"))
 (segment (start 189.165685 114.8) (end 189.4 114.565685) (width 0.2) (layer "F.Cu") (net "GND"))
 (segment (start 174.825 80.475) (end 174.825 92.338642) (width 0.2) (layer "F.Cu") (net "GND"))
 (segment (start 169.66 77.788) (end 170.672 78.8) (width 0.2) (layer "F.Cu") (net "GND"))
 (segment (start 170.672 78.8) (end 176.5 78.8) (width 0.2) (layer "F.Cu") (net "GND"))
 (segment (start 189.4 114.565685) (end 189.4 91.7) (width 0.2) (layer "F.Cu") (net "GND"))
 (segment (start 152.5 109.54) (end 157.76 114.8) (width 0.2) (layer "F.Cu") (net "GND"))
 (segment (start 119.69 66.492) (end 119.69 99) (width 0.2) (layer "F.Cu") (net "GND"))
 (segment (start 115.65 103.04) (end 115.65 102.5) (width 0.2) (layer "F.Cu") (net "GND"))
 (segment (start 149 100.96) (end 149 92.5) (width 0.2) (layer "F.Cu") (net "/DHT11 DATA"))
 (segment (start 149 90.135) (end 149 92.5) (width 0.2) (layer "F.Cu") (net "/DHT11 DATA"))
 (segment (start 152.5 104.46) (end 149 100.96) (width 0.2) (layer "F.Cu") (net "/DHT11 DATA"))
 (segment (start 160.335 78.8) (end 149 90.135) (width 0.2) (layer "F.Cu") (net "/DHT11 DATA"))
 (segment (start 160.335 81.34) (end 162.01 79.665) (width 0.2) (layer "F.Cu") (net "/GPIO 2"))
 (segment (start 146.5 95) (end 146.46 95) (width 0.2) (layer "F.Cu") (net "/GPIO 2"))
 (segment (start 146.5 87.581358) (end 146.5 95) (width 0.2) (layer "F.Cu") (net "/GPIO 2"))
 (segment (start 162.01 75.421358) (end 161.548642 74.96) (width 0.2) (layer "F.Cu") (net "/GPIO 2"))
 (segment (start 161.548642 74.96) (end 159.121358 74.96) (width 0.2) (layer "F.Cu") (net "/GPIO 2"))
 (segment (start 146.46 95) (end 141.04 100.42) (width 0.2) (layer "F.Cu") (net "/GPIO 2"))
 (segment (start 162.01 79.665) (end 162.01 75.421358) (width 0.2) (layer "F.Cu") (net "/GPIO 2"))
 (segment (start 159.121358 74.96) (end 146.5 87.581358) (width 0.2) (layer "F.Cu") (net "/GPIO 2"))
 (segment (start 153.55 104.025075) (end 152.934925 103.41) (width 0.2) (layer "F.Cu") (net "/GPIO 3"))
 (segment (start 139.140101 100.5) (end 140.460101 101.82) (width 0.2) (layer "F.Cu") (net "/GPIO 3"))
 (segment (start 149.4 100.794314) (end 149.4 94.815) (width 0.2) (layer "F.Cu") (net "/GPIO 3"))
 (segment (start 152.934925 105.51) (end 153.55 104.894925) (width 0.2) (layer "F.Cu") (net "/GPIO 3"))
 (segment (start 152.015686 103.41) (end 149.4 100.794314) (width 0.2) (layer "F.Cu") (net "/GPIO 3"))
 (segment (start 149.4 94.815) (end 160.335 83.88) (width 0.2) (layer "F.Cu") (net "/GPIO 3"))
 (segment (start 122 100.5) (end 139.140101 100.5) (width 0.2) (layer "F.Cu") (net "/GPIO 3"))
 (segment (start 153.55 104.894925) (end 153.55 104.025075) (width 0.2) (layer "F.Cu") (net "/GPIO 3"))
 (segment (start 152.934925 103.41) (end 152.015686 103.41) (width 0.2) (layer "F.Cu") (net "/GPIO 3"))
 (segment (start 140.460101 101.82) (end 148.375075 101.82) (width 0.2) (layer "F.Cu") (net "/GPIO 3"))
 (segment (start 152.065075 105.51) (end 152.934925 105.51) (width 0.2) (layer "F.Cu") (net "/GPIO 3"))
 (segment (start 148.375075 101.82) (end 152.065075 105.51) (width 0.2) (layer "F.Cu") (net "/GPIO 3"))
 (segment (start 162.41 79.830685) (end 162.41 75.255672) (width 0.2) (layer "F.Cu") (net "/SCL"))
 (segment (start 162.41 75.255672) (end 158.154328 71) (width 0.2) (layer "F.Cu") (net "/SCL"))
 (segment (start 160.335 86.42) (end 166.38 86.42) (width 0.2) (layer "F.Cu") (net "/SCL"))
 (segment (start 158.154328 71) (end 129.278 71) (width 0.2) (layer "F.Cu") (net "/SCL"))
 (segment (start 166.38 86.42) (end 180 100.04) (width 0.2) (layer "F.Cu") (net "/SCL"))
 (segment (start 162.01 84.745) (end 162.01 80.230685) (width 0.2) (layer "F.Cu") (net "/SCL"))
 (segment (start 162.01 80.230685) (end 162.41 79.830685) (width 0.2) (layer "F.Cu") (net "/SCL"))
 (segment (start 129.278 71) (end 124.77 66.492) (width 0.2) (layer "F.Cu") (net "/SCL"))
 (segment (start 160.335 86.42) (end 162.01 84.745) (width 0.2) (layer "F.Cu") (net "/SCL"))
 (segment (start 127.31 66.492) (end 130.207993 69.389993) (width 0.2) (layer "F.Cu") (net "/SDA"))
 (segment (start 166.38 88.96) (end 160.335 88.96) (width 0.2) (layer "F.Cu") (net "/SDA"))
 (segment (start 181.15 100.516346) (end 181.15 99.563654) (width 0.2) (layer "F.Cu") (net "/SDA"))
 (segment (start 179.523654 98.89) (end 165.495 84.861346) (width 0.2) (layer "F.Cu") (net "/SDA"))
 (segment (start 165.495 77.774986) (end 157.110007 69.389993) (width 0.2) (layer "F.Cu") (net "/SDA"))
 (segment (start 130.207993 69.389993) (end 157.110007 69.389993) (width 0.2) (layer "F.Cu") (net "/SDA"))
 (segment (start 127.31 66.492) (end 127.492 66.492) (width 0.2) (layer "F.Cu") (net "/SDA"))
 (segment (start 165.495 84.861346) (end 165.495 77.774986) (width 0.2) (layer "F.Cu") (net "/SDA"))
 (segment (start 127.5 66.5) (end 127.492 66.492) (width 0.2) (layer "F.Cu") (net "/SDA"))
 (segment (start 180.476346 98.89) (end 179.523654 98.89) (width 0.2) (layer "F.Cu") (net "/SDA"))
 (segment (start 160.335 88.96) (end 172.565 101.19) (width 0.2) (layer "F.Cu") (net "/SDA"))
 (segment (start 172.565 101.19) (end 180.476346 101.19) (width 0.2) (layer "F.Cu") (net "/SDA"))
 (segment (start 181.15 99.563654) (end 180.476346 98.89) (width 0.2) (layer "F.Cu") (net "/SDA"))
 (segment (start 180.476346 101.19) (end 181.15 100.516346) (width 0.2) (layer "F.Cu") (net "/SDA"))
 (segment (start 180 102.58) (end 166.38 88.96) (width 0.2) (layer "F.Cu") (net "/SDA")))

